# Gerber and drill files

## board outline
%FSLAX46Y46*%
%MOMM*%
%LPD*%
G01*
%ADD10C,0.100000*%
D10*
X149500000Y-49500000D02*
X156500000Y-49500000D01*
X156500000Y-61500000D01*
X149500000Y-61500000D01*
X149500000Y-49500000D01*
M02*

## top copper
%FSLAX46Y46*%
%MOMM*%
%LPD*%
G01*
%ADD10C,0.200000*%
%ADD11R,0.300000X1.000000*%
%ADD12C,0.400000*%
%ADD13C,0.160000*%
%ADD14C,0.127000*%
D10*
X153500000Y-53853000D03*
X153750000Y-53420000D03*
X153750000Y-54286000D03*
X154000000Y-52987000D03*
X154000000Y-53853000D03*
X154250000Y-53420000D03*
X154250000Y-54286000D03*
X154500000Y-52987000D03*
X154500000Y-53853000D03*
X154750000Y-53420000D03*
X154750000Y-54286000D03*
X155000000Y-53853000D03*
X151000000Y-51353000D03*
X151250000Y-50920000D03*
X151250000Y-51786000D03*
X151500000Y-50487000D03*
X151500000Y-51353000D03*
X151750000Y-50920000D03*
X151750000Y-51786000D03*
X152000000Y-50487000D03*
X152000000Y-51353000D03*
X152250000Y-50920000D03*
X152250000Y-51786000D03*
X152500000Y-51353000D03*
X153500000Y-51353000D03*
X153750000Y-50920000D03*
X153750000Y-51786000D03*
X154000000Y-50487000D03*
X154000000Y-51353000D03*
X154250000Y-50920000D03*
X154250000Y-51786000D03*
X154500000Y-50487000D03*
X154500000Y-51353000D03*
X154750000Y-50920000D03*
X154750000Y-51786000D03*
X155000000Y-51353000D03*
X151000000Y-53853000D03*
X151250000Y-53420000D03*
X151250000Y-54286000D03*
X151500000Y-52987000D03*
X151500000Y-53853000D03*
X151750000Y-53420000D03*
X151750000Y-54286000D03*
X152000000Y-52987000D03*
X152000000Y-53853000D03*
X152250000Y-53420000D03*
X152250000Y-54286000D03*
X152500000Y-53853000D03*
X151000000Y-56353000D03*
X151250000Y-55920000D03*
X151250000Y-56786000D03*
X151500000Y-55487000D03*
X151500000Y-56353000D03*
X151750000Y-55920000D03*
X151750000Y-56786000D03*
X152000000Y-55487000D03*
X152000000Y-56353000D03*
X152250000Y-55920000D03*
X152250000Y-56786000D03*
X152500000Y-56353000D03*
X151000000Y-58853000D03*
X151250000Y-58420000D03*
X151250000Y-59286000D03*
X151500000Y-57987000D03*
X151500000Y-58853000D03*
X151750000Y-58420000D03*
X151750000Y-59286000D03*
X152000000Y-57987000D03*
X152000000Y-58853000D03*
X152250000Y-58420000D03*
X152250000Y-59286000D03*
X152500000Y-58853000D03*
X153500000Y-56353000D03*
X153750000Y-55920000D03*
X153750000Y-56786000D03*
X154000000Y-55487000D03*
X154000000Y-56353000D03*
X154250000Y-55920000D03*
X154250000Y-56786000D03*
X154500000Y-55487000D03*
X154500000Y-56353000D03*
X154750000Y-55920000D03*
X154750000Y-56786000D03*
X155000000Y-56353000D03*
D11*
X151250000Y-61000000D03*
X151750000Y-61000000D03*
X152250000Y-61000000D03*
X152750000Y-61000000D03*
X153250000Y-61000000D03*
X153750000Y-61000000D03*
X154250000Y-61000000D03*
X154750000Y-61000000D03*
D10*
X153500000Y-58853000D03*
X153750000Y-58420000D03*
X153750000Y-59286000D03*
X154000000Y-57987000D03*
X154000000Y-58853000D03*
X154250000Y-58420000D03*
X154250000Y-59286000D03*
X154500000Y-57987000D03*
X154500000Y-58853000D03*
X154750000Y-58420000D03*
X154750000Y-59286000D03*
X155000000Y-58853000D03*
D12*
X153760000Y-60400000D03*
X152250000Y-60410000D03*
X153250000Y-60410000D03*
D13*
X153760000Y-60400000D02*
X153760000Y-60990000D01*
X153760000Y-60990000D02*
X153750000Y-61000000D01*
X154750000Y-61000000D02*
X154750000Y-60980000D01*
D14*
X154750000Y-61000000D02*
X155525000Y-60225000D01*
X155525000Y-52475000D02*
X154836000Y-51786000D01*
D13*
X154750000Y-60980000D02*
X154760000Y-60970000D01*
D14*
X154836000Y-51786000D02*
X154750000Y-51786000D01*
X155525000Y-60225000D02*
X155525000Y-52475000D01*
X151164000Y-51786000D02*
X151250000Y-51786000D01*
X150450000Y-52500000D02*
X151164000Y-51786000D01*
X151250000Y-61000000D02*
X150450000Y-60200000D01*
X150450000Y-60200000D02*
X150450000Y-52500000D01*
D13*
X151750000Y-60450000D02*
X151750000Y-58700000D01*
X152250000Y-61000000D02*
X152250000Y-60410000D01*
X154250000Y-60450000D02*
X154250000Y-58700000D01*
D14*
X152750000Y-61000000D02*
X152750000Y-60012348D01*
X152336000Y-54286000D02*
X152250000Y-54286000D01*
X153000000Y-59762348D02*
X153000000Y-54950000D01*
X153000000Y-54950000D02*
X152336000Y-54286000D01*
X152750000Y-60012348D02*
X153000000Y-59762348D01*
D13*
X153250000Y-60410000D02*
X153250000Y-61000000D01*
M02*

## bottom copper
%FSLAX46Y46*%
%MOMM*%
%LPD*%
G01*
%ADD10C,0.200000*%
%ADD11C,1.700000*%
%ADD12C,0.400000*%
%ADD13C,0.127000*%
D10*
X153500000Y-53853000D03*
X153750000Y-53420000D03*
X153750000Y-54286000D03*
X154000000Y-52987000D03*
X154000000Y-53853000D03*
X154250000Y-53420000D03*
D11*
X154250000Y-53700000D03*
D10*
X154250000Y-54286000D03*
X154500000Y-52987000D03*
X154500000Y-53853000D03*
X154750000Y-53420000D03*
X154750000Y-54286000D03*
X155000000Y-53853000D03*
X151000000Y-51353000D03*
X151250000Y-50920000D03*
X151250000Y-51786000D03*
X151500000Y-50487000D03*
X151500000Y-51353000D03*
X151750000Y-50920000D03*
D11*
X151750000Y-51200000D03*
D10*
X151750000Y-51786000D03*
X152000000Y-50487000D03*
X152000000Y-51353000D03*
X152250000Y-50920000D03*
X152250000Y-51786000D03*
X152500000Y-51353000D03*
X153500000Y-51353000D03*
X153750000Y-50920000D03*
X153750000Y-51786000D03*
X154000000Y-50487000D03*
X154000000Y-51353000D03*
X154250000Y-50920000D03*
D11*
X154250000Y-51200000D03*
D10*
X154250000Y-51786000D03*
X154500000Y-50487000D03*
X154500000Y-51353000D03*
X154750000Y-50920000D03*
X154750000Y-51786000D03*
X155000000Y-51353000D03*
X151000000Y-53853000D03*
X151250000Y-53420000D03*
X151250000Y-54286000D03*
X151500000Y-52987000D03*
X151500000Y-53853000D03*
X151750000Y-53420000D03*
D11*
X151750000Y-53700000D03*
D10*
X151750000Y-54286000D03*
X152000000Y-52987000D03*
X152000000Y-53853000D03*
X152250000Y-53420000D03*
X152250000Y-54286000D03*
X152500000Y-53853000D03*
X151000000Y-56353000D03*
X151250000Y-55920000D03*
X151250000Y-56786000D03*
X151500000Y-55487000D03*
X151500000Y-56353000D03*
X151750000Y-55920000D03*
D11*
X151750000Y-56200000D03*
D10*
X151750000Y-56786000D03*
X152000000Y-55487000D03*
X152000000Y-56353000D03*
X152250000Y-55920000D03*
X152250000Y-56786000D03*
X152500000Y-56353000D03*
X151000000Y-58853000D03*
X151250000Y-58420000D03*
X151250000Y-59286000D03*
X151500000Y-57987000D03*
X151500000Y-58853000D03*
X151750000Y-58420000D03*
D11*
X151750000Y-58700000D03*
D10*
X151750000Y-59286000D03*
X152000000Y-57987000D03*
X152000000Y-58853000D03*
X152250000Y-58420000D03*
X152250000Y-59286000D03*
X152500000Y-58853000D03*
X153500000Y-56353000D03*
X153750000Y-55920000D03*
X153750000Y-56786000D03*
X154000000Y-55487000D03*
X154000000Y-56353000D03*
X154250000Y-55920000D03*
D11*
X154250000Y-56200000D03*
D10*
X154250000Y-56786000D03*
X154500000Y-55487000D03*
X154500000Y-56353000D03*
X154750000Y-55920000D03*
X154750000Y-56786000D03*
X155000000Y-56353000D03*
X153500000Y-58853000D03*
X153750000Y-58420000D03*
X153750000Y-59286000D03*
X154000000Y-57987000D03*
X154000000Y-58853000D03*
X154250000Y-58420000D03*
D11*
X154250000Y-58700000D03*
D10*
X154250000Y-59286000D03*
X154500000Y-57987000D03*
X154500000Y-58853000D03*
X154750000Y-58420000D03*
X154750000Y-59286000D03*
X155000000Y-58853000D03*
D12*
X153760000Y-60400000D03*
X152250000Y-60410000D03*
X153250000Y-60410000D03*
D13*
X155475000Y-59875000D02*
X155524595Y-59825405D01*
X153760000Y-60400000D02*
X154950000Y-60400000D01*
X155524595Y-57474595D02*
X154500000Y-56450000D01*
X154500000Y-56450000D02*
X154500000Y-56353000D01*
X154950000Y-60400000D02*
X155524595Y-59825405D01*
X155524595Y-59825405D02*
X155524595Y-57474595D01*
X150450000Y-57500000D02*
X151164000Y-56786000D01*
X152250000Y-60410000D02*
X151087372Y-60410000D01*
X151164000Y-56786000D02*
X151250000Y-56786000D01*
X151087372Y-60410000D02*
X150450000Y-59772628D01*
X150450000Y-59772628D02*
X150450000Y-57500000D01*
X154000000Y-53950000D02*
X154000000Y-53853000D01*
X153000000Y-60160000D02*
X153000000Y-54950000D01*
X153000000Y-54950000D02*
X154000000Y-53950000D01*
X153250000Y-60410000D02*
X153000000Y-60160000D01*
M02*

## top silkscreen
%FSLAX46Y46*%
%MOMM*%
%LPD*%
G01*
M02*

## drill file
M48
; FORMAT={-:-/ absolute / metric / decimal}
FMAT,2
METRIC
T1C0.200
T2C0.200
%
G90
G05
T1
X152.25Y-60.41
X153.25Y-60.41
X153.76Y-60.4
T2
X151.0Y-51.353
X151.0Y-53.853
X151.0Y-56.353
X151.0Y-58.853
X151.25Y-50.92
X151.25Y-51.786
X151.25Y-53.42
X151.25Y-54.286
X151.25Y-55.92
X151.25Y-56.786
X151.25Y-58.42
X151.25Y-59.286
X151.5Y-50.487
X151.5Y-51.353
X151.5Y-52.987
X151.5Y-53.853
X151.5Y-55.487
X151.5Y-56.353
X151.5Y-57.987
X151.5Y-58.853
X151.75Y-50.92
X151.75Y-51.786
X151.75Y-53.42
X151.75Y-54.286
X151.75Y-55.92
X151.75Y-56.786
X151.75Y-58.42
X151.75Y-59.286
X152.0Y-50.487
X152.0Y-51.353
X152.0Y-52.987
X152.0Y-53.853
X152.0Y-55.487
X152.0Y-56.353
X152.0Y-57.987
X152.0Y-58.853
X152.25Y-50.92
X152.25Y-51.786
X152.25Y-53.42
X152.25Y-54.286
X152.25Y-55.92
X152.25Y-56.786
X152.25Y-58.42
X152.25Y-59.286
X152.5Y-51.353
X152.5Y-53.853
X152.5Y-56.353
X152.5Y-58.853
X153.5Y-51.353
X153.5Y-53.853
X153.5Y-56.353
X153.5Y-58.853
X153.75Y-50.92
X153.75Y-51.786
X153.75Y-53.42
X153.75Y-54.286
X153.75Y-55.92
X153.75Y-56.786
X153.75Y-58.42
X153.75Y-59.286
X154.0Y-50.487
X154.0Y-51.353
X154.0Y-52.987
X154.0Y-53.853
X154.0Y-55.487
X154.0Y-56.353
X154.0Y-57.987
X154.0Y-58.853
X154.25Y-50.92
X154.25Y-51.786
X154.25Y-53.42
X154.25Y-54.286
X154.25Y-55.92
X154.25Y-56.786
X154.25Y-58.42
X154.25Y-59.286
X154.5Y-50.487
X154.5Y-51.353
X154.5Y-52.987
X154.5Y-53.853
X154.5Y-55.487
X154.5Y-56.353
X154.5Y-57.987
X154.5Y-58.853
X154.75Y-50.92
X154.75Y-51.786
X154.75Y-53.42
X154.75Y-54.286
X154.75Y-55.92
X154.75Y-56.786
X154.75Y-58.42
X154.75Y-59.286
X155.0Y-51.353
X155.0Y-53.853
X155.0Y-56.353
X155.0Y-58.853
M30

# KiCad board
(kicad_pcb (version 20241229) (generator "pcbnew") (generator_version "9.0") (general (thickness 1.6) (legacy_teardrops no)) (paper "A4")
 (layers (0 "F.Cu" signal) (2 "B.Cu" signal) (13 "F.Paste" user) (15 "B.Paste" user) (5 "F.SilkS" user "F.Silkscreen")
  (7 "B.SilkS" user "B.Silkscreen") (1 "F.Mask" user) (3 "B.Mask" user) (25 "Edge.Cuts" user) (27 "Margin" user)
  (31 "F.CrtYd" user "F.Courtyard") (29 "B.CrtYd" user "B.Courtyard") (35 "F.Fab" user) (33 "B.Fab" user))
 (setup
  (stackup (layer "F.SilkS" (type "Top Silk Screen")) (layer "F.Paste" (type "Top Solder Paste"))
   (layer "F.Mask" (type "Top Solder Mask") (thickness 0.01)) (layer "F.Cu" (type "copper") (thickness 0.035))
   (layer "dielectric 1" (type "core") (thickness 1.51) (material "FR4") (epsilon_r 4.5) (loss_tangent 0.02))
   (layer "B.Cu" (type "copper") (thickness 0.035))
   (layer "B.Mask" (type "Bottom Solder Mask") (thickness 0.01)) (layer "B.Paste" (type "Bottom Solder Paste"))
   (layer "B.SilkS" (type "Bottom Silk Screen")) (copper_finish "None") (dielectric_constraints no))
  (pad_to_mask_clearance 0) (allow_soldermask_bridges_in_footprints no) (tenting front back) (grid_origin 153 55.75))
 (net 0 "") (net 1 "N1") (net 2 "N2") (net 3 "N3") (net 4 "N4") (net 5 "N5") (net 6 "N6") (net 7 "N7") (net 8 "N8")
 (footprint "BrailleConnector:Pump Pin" (layer "F.Cu") (at 154.25 53.7)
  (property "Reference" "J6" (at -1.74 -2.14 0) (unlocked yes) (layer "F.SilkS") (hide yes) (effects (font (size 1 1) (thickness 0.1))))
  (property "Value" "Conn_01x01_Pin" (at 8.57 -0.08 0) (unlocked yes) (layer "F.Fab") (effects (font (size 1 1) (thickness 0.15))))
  (pad "1" thru_hole circle (at -0.75 0.153) (size 0.2 0.2) (drill 0.2) (layers "*.Cu" "*.Mask") (remove_unused_layers no) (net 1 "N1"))
  (pad "1" thru_hole circle (at -0.5 -0.28) (size 0.2 0.2) (drill 0.2) (layers "*.Cu" "*.Mask") (remove_unused_layers no) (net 1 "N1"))
  (pad "1" thru_hole circle (at -0.5 0.586) (size 0.2 0.2) (drill 0.2) (layers "*.Cu" "*.Mask") (remove_unused_layers no) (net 1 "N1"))
  (pad "1" thru_hole circle (at -0.25 -0.713) (size 0.2 0.2) (drill 0.2) (layers "*.Cu" "*.Mask") (remove_unused_layers no) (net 1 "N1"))
  (pad "1" thru_hole circle (at -0.25 0.153) (size 0.2 0.2) (drill 0.2) (layers "*.Cu" "*.Mask") (remove_unused_layers no) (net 1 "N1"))
  (pad "1" thru_hole circle (at 0 -0.28) (size 0.2 0.2) (drill 0.2) (layers "*.Cu" "*.Mask") (remove_unused_layers no) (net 1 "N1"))
  (pad "1" smd circle (at 0 0) (size 1.7 1.7) (layers "B.Cu" "B.Mask") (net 1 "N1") (solder_mask_margin 0) (solder_paste_margin 0)
   (clearance 0))
  (pad "1" thru_hole circle (at 0 0.586) (size 0.2 0.2) (drill 0.2) (layers "*.Cu" "*.Mask") (remove_unused_layers no) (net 1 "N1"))
  (pad "1" thru_hole circle (at 0.25 -0.713) (size 0.2 0.2) (drill 0.2) (layers "*.Cu" "*.Mask") (remove_unused_layers no) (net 1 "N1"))
  (pad "1" thru_hole circle (at 0.25 0.153) (size 0.2 0.2) (drill 0.2) (layers "*.Cu" "*.Mask") (remove_unused_layers no) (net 1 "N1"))
  (pad "1" thru_hole circle (at 0.5 -0.28) (size 0.2 0.2) (drill 0.2) (layers "*.Cu" "*.Mask") (remove_unused_layers no) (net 1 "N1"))
  (pad "1" thru_hole circle (at 0.5 0.586) (size 0.2 0.2) (drill 0.2) (layers "*.Cu" "*.Mask") (remove_unused_layers no) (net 1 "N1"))
  (pad "1" thru_hole circle (at 0.75 0.153) (size 0.2 0.2) (drill 0.2) (layers "*.Cu" "*.Mask") (remove_unused_layers no) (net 1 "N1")))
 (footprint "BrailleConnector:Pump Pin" (layer "F.Cu") (at 151.75 51.2)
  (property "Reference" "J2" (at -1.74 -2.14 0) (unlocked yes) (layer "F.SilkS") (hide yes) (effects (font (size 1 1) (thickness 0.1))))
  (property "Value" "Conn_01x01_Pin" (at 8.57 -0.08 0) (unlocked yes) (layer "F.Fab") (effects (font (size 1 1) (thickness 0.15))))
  (pad "1" thru_hole circle (at -0.75 0.153) (size 0.2 0.2) (drill 0.2) (layers "*.Cu" "*.Mask") (remove_unused_layers no) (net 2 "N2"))
  (pad "1" thru_hole circle (at -0.5 -0.28) (size 0.2 0.2) (drill 0.2) (layers "*.Cu" "*.Mask") (remove_unused_layers no) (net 2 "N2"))
  (pad "1" thru_hole circle (at -0.5 0.586) (size 0.2 0.2) (drill 0.2) (layers "*.Cu" "*.Mask") (remove_unused_layers no) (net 2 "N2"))
  (pad "1" thru_hole circle (at -0.25 -0.713) (size 0.2 0.2) (drill 0.2) (layers "*.Cu" "*.Mask") (remove_unused_layers no) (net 2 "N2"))
  (pad "1" thru_hole circle (at -0.25 0.153) (size 0.2 0.2) (drill 0.2) (layers "*.Cu" "*.Mask") (remove_unused_layers no) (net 2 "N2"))
  (pad "1" thru_hole circle (at 0 -0.28) (size 0.2 0.2) (drill 0.2) (layers "*.Cu" "*.Mask") (remove_unused_layers no) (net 2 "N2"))
  (pad "1" smd circle (at 0 0) (size 1.7 1.7) (layers "B.Cu" "B.Mask") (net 2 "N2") (solder_mask_margin 0) (solder_paste_margin 0)
   (clearance 0))
  (pad "1" thru_hole circle (at 0 0.586) (size 0.2 0.2) (drill 0.2) (layers "*.Cu" "*.Mask") (remove_unused_layers no) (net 2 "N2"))
  (pad "1" thru_hole circle (at 0.25 -0.713) (size 0.2 0.2) (drill 0.2) (layers "*.Cu" "*.Mask") (remove_unused_layers no) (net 2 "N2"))
  (pad "1" thru_hole circle (at 0.25 0.153) (size 0.2 0.2) (drill 0.2) (layers "*.Cu" "*.Mask") (remove_unused_layers no) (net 2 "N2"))
  (pad "1" thru_hole circle (at 0.5 -0.28) (size 0.2 0.2) (drill 0.2) (layers "*.Cu" "*.Mask") (remove_unused_layers no) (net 2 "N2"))
  (pad "1" thru_hole circle (at 0.5 0.586) (size 0.2 0.2) (drill 0.2) (layers "*.Cu" "*.Mask") (remove_unused_layers no) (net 2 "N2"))
  (pad "1" thru_hole circle (at 0.75 0.153) (size 0.2 0.2) (drill 0.2) (layers "*.Cu" "*.Mask") (remove_unused_layers no) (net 2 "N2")))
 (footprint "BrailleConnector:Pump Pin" (layer "F.Cu") (at 154.25 51.2)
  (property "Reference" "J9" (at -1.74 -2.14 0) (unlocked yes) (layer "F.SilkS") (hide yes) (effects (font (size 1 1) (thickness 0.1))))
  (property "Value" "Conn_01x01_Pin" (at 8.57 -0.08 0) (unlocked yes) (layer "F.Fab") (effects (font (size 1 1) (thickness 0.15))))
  (pad "1" thru_hole circle (at -0.75 0.153) (size 0.2 0.2) (drill 0.2) (layers "*.Cu" "*.Mask") (remove_unused_layers no) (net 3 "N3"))
  (pad "1" thru_hole circle (at -0.5 -0.28) (size 0.2 0.2) (drill 0.2) (layers "*.Cu" "*.Mask") (remove_unused_layers no) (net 3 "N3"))
  (pad "1" thru_hole circle (at -0.5 0.586) (size 0.2 0.2) (drill 0.2) (layers "*.Cu" "*.Mask") (remove_unused_layers no) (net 3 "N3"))
  (pad "1" thru_hole circle (at -0.25 -0.713) (size 0.2 0.2) (drill 0.2) (layers "*.Cu" "*.Mask") (remove_unused_layers no) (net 3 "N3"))
  (pad "1" thru_hole circle (at -0.25 0.153) (size 0.2 0.2) (drill 0.2) (layers "*.Cu" "*.Mask") (remove_unused_layers no) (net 3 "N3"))
  (pad "1" thru_hole circle (at 0 -0.28) (size 0.2 0.2) (drill 0.2) (layers "*.Cu" "*.Mask") (remove_unused_layers no) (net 3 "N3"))
  (pad "1" smd circle (at 0 0) (size 1.7 1.7) (layers "B.Cu" "B.Mask") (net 3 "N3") (solder_mask_margin 0) (solder_paste_margin 0)
   (clearance 0))
  (pad "1" thru_hole circle (at 0 0.586) (size 0.2 0.2) (drill 0.2) (layers "*.Cu" "*.Mask") (remove_unused_layers no) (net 3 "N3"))
  (pad "1" thru_hole circle (at 0.25 -0.713) (size 0.2 0.2) (drill 0.2) (layers "*.Cu" "*.Mask") (remove_unused_layers no) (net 3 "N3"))
  (pad "1" thru_hole circle (at 0.25 0.153) (size 0.2 0.2) (drill 0.2) (layers "*.Cu" "*.Mask") (remove_unused_layers no) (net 3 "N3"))
  (pad "1" thru_hole circle (at 0.5 -0.28) (size 0.2 0.2) (drill 0.2) (layers "*.Cu" "*.Mask") (remove_unused_layers no) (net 3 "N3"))
  (pad "1" thru_hole circle (at 0.5 0.586) (size 0.2 0.2) (drill 0.2) (layers "*.Cu" "*.Mask") (remove_unused_layers no) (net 3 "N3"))
  (pad "1" thru_hole circle (at 0.75 0.153) (size 0.2 0.2) (drill 0.2) (layers "*.Cu" "*.Mask") (remove_unused_layers no) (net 3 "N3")))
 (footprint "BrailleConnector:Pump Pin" (layer "F.Cu") (at 151.75 53.7)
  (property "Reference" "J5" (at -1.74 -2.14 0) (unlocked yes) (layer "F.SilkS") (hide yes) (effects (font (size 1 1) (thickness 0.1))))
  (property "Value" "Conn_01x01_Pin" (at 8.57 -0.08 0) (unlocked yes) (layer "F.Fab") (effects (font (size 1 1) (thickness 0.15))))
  (pad "1" thru_hole circle (at -0.75 0.153) (size 0.2 0.2) (drill 0.2) (layers "*.Cu" "*.Mask") (remove_unused_layers no) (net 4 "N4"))
  (pad "1" thru_hole circle (at -0.5 -0.28) (size 0.2 0.2) (drill 0.2) (layers "*.Cu" "*.Mask") (remove_unused_layers no) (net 4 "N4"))
  (pad "1" thru_hole circle (at -0.5 0.586) (size 0.2 0.2) (drill 0.2) (layers "*.Cu" "*.Mask") (remove_unused_layers no) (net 4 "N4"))
  (pad "1" thru_hole circle (at -0.25 -0.713) (size 0.2 0.2) (drill 0.2) (layers "*.Cu" "*.Mask") (remove_unused_layers no) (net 4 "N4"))
  (pad "1" thru_hole circle (at -0.25 0.153) (size 0.2 0.2) (drill 0.2) (layers "*.Cu" "*.Mask") (remove_unused_layers no) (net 4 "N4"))
  (pad "1" thru_hole circle (at 0 -0.28) (size 0.2 0.2) (drill 0.2) (layers "*.Cu" "*.Mask") (remove_unused_layers no) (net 4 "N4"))
  (pad "1" smd circle (at 0 0) (size 1.7 1.7) (layers "B.Cu" "B.Mask") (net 4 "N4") (solder_mask_margin 0) (solder_paste_margin 0)
   (clearance 0))
  (pad "1" thru_hole circle (at 0 0.586) (size 0.2 0.2) (drill 0.2) (layers "*.Cu" "*.Mask") (remove_unused_layers no) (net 4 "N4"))
  (pad "1" thru_hole circle (at 0.25 -0.713) (size 0.2 0.2) (drill 0.2) (layers "*.Cu" "*.Mask") (remove_unused_layers no) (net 4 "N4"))
  (pad "1" thru_hole circle (at 0.25 0.153) (size 0.2 0.2) (drill 0.2) (layers "*.Cu" "*.Mask") (remove_unused_layers no) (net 4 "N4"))
  (pad "1" thru_hole circle (at 0.5 -0.28) (size 0.2 0.2) (drill 0.2) (layers "*.Cu" "*.Mask") (remove_unused_layers no) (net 4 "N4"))
  (pad "1" thru_hole circle (at 0.5 0.586) (size 0.2 0.2) (drill 0.2) (layers "*.Cu" "*.Mask") (remove_unused_layers no) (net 4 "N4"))
  (pad "1" thru_hole circle (at 0.75 0.153) (size 0.2 0.2) (drill 0.2) (layers "*.Cu" "*.Mask") (remove_unused_layers no) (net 4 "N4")))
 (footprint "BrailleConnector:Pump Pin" (layer "F.Cu") (at 151.75 56.2)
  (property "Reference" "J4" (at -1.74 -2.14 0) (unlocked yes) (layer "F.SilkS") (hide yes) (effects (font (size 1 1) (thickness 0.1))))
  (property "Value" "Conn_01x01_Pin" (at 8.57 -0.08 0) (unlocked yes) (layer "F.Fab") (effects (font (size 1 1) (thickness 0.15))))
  (pad "1" thru_hole circle (at -0.75 0.153) (size 0.2 0.2) (drill 0.2) (layers "*.Cu" "*.Mask") (remove_unused_layers no) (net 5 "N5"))
  (pad "1" thru_hole circle (at -0.5 -0.28) (size 0.2 0.2) (drill 0.2) (layers "*.Cu" "*.Mask") (remove_unused_layers no) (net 5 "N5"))
  (pad "1" thru_hole circle (at -0.5 0.586) (size 0.2 0.2) (drill 0.2) (layers "*.Cu" "*.Mask") (remove_unused_layers no) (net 5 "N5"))
  (pad "1" thru_hole circle (at -0.25 -0.713) (size 0.2 0.2) (drill 0.2) (layers "*.Cu" "*.Mask") (remove_unused_layers no) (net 5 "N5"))
  (pad "1" thru_hole circle (at -0.25 0.153) (size 0.2 0.2) (drill 0.2) (layers "*.Cu" "*.Mask") (remove_unused_layers no) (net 5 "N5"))
  (pad "1" thru_hole circle (at 0 -0.28) (size 0.2 0.2) (drill 0.2) (layers "*.Cu" "*.Mask") (remove_unused_layers no) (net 5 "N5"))
  (pad "1" smd circle (at 0 0) (size 1.7 1.7) (layers "B.Cu" "B.Mask") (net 5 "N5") (solder_mask_margin 0) (solder_paste_margin 0)
   (clearance 0))
  (pad "1" thru_hole circle (at 0 0.586) (size 0.2 0.2) (drill 0.2) (layers "*.Cu" "*.Mask") (remove_unused_layers no) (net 5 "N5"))
  (pad "1" thru_hole circle (at 0.25 -0.713) (size 0.2 0.2) (drill 0.2) (layers "*.Cu" "*.Mask") (remove_unused_layers no) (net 5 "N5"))
  (pad "1" thru_hole circle (at 0.25 0.153) (size 0.2 0.2) (drill 0.2) (layers "*.Cu" "*.Mask") (remove_unused_layers no) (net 5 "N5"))
  (pad "1" thru_hole circle (at 0.5 -0.28) (size 0.2 0.2) (drill 0.2) (layers "*.Cu" "*.Mask") (remove_unused_layers no) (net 5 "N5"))
  (pad "1" thru_hole circle (at 0.5 0.586) (size 0.2 0.2) (drill 0.2) (layers "*.Cu" "*.Mask") (remove_unused_layers no) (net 5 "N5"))
  (pad "1" thru_hole circle (at 0.75 0.153) (size 0.2 0.2) (drill 0.2) (layers "*.Cu" "*.Mask") (remove_unused_layers no) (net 5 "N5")))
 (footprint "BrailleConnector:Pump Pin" (layer "F.Cu") (at 151.75 58.7)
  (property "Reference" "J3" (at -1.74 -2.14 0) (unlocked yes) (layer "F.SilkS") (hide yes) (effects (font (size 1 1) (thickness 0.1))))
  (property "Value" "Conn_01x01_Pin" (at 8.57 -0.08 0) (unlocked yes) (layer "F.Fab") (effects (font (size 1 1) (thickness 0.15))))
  (pad "1" thru_hole circle (at -0.75 0.153) (size 0.2 0.2) (drill 0.2) (layers "*.Cu" "*.Mask") (remove_unused_layers no) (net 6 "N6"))
  (pad "1" thru_hole circle (at -0.5 -0.28) (size 0.2 0.2) (drill 0.2) (layers "*.Cu" "*.Mask") (remove_unused_layers no) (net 6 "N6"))
  (pad "1" thru_hole circle (at -0.5 0.586) (size 0.2 0.2) (drill 0.2) (layers "*.Cu" "*.Mask") (remove_unused_layers no) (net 6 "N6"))
  (pad "1" thru_hole circle (at -0.25 -0.713) (size 0.2 0.2) (drill 0.2) (layers "*.Cu" "*.Mask") (remove_unused_layers no) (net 6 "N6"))
  (pad "1" thru_hole circle (at -0.25 0.153) (size 0.2 0.2) (drill 0.2) (layers "*.Cu" "*.Mask") (remove_unused_layers no) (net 6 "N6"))
  (pad "1" thru_hole circle (at 0 -0.28) (size 0.2 0.2) (drill 0.2) (layers "*.Cu" "*.Mask") (remove_unused_layers no) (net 6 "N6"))
  (pad "1" smd circle (at 0 0) (size 1.7 1.7) (layers "B.Cu" "B.Mask") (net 6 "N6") (solder_mask_margin 0) (solder_paste_margin 0)
   (clearance 0))
  (pad "1" thru_hole circle (at 0 0.586) (size 0.2 0.2) (drill 0.2) (layers "*.Cu" "*.Mask") (remove_unused_layers no) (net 6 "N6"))
  (pad "1" thru_hole circle (at 0.25 -0.713) (size 0.2 0.2) (drill 0.2) (layers "*.Cu" "*.Mask") (remove_unused_layers no) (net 6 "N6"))
  (pad "1" thru_hole circle (at 0.25 0.153) (size 0.2 0.2) (drill 0.2) (layers "*.Cu" "*.Mask") (remove_unused_layers no) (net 6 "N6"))
  (pad "1" thru_hole circle (at 0.5 -0.28) (size 0.2 0.2) (drill 0.2) (layers "*.Cu" "*.Mask") (remove_unused_layers no) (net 6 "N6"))
  (pad "1" thru_hole circle (at 0.5 0.586) (size 0.2 0.2) (drill 0.2) (layers "*.Cu" "*.Mask") (remove_unused_layers no) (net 6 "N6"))
  (pad "1" thru_hole circle (at 0.75 0.153) (size 0.2 0.2) (drill 0.2) (layers "*.Cu" "*.Mask") (remove_unused_layers no) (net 6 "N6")))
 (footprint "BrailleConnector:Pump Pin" (layer "F.Cu") (at 154.25 56.2)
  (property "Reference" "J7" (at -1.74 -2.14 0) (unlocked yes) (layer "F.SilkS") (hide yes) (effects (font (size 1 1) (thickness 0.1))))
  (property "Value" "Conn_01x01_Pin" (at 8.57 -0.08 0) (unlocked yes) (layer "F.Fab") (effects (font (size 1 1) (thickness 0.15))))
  (pad "1" thru_hole circle (at -0.75 0.153) (size 0.2 0.2) (drill 0.2) (layers "*.Cu" "*.Mask") (remove_unused_layers no) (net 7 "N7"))
  (pad "1" thru_hole circle (at -0.5 -0.28) (size 0.2 0.2) (drill 0.2) (layers "*.Cu" "*.Mask") (remove_unused_layers no) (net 7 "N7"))
  (pad "1" thru_hole circle (at -0.5 0.586) (size 0.2 0.2) (drill 0.2) (layers "*.Cu" "*.Mask") (remove_unused_layers no) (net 7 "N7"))
  (pad "1" thru_hole circle (at -0.25 -0.713) (size 0.2 0.2) (drill 0.2) (layers "*.Cu" "*.Mask") (remove_unused_layers no) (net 7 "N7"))
  (pad "1" thru_hole circle (at -0.25 0.153) (size 0.2 0.2) (drill 0.2) (layers "*.Cu" "*.Mask") (remove_unused_layers no) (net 7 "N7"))
  (pad "1" thru_hole circle (at 0 -0.28) (size 0.2 0.2) (drill 0.2) (layers "*.Cu" "*.Mask") (remove_unused_layers no) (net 7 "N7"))
  (pad "1" smd circle (at 0 0) (size 1.7 1.7) (layers "B.Cu" "B.Mask") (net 7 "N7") (solder_mask_margin 0) (solder_paste_margin 0)
   (clearance 0))
  (pad "1" thru_hole circle (at 0 0.586) (size 0.2 0.2) (drill 0.2) (layers "*.Cu" "*.Mask") (remove_unused_layers no) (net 7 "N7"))
  (pad "1" thru_hole circle (at 0.25 -0.713) (size 0.2 0.2) (drill 0.2) (layers "*.Cu" "*.Mask") (remove_unused_layers no) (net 7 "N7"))
  (pad "1" thru_hole circle (at 0.25 0.153) (size 0.2 0.2) (drill 0.2) (layers "*.Cu" "*.Mask") (remove_unused_layers no) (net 7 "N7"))
  (pad "1" thru_hole circle (at 0.5 -0.28) (size 0.2 0.2) (drill 0.2) (layers "*.Cu" "*.Mask") (remove_unused_layers no) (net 7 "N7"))
  (pad "1" thru_hole circle (at 0.5 0.586) (size 0.2 0.2) (drill 0.2) (layers "*.Cu" "*.Mask") (remove_unused_layers no) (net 7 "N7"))
  (pad "1" thru_hole circle (at 0.75 0.153) (size 0.2 0.2) (drill 0.2) (layers "*.Cu" "*.Mask") (remove_unused_layers no) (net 7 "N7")))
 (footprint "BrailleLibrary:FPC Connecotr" (layer "F.Cu") (at 153 61 90)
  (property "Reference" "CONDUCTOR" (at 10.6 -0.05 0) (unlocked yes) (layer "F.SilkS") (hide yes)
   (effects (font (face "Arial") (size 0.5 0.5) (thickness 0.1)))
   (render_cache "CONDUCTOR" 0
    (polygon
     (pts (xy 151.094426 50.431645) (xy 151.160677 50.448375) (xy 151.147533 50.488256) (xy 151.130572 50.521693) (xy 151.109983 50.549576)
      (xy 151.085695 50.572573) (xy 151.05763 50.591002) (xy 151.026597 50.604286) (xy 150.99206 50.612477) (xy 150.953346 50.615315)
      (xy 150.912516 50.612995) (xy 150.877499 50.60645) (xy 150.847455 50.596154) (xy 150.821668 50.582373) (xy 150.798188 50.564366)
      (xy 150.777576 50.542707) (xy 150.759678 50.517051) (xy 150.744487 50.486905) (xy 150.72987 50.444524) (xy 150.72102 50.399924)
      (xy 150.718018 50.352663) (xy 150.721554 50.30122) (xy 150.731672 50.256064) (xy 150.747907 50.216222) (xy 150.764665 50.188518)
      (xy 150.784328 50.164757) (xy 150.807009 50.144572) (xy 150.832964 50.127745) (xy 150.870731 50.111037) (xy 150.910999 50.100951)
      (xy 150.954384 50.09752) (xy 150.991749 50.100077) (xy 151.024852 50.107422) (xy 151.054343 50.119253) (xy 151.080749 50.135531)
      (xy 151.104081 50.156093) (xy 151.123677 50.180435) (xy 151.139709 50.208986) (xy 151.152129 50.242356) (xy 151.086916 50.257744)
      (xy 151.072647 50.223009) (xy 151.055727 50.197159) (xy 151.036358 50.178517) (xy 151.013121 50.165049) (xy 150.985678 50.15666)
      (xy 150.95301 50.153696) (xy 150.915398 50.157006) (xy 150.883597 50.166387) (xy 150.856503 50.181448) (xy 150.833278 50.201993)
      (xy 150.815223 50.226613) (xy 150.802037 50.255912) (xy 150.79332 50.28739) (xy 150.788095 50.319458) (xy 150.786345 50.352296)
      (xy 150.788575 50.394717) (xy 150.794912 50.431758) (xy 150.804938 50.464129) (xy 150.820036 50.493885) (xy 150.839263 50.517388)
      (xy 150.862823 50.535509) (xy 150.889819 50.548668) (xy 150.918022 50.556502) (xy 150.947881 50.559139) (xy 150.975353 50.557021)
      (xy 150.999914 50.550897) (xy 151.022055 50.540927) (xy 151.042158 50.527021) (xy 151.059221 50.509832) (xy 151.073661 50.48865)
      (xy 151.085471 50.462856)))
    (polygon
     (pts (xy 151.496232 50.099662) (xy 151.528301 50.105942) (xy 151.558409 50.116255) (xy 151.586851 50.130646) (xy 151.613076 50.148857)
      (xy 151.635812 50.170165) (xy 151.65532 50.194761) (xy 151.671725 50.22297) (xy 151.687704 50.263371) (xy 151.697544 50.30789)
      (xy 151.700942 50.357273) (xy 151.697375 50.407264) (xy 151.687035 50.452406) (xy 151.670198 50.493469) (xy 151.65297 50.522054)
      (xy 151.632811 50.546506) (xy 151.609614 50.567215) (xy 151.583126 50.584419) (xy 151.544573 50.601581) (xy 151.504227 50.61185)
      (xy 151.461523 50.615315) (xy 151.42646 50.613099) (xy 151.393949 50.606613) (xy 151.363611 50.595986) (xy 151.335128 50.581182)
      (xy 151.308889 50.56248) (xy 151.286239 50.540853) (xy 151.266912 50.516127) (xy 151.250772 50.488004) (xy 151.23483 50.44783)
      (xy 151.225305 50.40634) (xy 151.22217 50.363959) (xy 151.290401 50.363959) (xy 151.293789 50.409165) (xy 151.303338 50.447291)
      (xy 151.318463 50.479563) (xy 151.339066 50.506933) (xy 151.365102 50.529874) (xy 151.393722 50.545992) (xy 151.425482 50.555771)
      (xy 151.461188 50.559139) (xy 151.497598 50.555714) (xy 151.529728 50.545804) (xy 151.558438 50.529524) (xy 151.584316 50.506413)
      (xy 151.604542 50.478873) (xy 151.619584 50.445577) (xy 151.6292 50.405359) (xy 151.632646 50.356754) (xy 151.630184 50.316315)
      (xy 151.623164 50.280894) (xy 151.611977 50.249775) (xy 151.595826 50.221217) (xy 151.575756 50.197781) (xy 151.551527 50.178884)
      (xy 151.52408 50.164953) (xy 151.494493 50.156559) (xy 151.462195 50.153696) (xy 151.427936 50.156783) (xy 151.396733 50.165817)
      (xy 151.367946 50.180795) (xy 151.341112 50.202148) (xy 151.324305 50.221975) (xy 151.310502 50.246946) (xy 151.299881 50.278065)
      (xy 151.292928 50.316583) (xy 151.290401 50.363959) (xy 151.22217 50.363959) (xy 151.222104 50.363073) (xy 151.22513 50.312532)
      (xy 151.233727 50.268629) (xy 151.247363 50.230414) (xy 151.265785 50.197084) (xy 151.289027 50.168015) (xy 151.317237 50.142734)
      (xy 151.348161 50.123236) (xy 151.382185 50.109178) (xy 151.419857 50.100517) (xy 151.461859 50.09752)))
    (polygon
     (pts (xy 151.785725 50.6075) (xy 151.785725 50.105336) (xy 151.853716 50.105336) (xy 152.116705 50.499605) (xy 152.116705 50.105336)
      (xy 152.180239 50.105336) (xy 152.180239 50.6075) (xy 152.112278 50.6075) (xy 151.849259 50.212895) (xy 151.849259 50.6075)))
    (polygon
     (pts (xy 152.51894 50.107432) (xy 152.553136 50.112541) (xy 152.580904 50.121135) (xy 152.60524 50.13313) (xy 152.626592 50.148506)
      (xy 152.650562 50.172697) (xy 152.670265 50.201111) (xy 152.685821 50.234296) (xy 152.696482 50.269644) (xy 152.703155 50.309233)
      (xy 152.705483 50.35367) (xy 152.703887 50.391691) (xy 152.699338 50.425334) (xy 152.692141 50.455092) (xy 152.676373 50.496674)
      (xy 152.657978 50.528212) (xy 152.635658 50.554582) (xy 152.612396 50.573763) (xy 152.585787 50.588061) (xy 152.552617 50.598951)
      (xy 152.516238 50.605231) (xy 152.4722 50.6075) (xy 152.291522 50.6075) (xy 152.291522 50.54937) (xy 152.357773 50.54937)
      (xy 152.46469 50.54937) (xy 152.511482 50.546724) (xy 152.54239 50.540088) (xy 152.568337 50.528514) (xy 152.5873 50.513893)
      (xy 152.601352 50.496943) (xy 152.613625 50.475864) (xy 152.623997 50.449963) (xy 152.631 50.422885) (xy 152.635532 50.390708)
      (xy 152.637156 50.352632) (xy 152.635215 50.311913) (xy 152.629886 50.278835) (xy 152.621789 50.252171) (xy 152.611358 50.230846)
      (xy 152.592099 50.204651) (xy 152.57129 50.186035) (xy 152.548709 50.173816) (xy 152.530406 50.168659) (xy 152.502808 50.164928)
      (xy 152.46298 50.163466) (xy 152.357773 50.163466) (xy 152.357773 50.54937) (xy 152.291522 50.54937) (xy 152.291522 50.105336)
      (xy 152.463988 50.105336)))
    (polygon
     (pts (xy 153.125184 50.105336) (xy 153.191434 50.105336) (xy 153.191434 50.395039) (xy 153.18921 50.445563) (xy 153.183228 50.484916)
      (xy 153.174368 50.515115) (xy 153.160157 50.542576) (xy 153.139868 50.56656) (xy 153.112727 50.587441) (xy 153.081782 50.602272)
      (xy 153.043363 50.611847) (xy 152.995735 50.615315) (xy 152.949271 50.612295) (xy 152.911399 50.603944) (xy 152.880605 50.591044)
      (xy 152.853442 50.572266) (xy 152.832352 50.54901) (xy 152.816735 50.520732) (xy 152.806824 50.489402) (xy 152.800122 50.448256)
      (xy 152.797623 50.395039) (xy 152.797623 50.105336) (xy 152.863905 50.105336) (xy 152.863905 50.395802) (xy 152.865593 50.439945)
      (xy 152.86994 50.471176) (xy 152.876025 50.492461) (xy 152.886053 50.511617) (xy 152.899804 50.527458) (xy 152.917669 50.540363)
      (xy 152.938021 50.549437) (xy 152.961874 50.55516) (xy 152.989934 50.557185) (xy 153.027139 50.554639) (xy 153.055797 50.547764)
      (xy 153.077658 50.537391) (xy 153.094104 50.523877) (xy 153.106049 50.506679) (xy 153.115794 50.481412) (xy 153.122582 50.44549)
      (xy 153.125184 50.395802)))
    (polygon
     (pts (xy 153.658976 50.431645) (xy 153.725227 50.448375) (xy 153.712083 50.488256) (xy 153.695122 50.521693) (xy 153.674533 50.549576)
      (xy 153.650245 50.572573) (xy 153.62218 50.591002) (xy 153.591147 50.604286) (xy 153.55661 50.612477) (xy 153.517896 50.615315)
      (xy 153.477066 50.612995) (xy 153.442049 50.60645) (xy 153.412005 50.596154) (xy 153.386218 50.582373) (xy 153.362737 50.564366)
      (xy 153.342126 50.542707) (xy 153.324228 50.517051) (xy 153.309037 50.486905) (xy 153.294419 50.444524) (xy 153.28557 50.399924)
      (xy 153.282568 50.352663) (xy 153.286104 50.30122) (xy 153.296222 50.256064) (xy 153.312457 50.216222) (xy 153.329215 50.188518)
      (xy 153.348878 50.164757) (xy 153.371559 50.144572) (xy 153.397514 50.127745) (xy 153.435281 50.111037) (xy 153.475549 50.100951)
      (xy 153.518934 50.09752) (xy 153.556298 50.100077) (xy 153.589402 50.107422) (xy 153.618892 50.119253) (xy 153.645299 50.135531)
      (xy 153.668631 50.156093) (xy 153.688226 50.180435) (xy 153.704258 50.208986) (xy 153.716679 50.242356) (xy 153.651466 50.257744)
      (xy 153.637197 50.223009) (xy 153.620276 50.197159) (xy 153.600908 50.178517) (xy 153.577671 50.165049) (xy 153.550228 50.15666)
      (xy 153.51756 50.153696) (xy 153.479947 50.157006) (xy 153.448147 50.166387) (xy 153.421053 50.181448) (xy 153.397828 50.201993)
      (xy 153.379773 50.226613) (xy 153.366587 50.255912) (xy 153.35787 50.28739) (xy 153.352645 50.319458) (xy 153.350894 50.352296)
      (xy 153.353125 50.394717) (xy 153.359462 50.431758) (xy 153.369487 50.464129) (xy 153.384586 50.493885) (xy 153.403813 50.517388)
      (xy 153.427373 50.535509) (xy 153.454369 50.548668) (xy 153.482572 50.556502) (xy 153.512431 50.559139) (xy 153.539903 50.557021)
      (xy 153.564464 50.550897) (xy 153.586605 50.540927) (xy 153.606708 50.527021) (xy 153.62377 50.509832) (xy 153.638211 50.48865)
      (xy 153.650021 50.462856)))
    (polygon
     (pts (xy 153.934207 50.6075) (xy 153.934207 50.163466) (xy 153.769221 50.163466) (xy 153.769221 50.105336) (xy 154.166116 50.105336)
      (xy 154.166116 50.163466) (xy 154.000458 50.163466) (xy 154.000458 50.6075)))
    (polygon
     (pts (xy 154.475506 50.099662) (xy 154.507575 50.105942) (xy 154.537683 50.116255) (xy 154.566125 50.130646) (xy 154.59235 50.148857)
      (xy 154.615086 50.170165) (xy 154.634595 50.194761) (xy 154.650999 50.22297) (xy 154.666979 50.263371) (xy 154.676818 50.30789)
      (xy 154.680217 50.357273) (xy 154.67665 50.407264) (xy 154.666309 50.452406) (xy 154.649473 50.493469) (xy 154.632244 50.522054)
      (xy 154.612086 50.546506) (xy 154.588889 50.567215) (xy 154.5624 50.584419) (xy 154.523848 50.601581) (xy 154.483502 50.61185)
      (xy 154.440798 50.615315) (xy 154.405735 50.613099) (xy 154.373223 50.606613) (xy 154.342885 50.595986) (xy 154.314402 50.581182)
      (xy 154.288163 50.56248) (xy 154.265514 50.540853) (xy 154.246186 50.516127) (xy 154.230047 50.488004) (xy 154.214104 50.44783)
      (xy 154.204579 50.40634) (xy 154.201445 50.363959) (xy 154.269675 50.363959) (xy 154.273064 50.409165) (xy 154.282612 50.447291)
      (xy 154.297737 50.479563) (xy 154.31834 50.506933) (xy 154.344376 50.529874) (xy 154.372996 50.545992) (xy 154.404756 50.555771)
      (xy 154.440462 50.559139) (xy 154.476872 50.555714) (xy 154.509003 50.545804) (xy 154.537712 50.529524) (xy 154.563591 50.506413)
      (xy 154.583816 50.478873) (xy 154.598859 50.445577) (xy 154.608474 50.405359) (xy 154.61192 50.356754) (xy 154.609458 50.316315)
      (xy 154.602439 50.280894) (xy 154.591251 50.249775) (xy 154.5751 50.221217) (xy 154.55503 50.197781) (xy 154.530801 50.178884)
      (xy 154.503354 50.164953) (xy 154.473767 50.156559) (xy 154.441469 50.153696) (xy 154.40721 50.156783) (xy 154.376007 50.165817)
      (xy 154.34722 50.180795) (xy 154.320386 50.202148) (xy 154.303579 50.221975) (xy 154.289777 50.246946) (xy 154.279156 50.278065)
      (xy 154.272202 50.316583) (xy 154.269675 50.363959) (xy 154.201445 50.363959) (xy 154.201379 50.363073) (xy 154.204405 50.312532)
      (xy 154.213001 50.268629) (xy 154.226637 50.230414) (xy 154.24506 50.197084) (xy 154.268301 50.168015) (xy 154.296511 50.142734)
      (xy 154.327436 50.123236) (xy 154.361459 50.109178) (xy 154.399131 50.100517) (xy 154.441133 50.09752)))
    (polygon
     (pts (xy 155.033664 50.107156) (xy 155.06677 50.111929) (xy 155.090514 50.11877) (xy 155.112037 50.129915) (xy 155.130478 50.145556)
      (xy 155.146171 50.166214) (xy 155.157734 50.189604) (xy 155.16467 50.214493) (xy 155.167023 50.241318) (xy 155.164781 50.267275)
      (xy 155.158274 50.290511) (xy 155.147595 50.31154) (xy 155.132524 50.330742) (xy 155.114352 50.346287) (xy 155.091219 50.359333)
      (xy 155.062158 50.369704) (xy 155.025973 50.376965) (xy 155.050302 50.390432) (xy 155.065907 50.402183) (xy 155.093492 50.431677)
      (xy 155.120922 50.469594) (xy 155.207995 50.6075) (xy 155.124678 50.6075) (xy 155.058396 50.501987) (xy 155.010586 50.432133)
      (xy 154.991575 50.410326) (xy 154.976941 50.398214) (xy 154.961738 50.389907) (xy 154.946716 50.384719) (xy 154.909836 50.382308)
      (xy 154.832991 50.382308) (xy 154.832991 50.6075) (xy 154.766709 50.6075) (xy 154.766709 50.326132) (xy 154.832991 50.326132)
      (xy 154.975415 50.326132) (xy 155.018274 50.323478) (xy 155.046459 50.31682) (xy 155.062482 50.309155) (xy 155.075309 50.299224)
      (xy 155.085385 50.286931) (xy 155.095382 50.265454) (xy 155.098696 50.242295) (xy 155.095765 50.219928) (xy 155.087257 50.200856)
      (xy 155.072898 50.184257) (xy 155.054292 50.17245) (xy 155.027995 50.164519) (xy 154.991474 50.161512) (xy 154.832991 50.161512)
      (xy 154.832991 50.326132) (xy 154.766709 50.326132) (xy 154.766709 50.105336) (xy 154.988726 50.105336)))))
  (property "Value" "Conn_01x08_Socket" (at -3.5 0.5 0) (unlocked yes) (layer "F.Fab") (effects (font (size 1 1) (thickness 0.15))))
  (pad "1" smd rect (at 0 -1.75 90) (size 1 0.3) (layers "F.Cu" "F.Mask" "F.Paste") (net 2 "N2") (thermal_bridge_angle 45))
  (pad "2" smd rect (at 0 -1.25 90) (size 1 0.3) (layers "F.Cu" "F.Mask" "F.Paste") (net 6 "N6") (thermal_bridge_angle 45))
  (pad "3" smd rect (at 0 -0.75 90) (size 1 0.3) (layers "F.Cu" "F.Mask" "F.Paste") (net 5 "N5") (thermal_bridge_angle 45))
  (pad "4" smd rect (at 0 -0.25 90) (size 1 0.3) (layers "F.Cu" "F.Mask" "F.Paste") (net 4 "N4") (thermal_bridge_angle 45))
  (pad "5" smd rect (at 0 0.25 90) (size 1 0.3) (layers "F.Cu" "F.Mask" "F.Paste") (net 1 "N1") (thermal_bridge_angle 45))
  (pad "6" smd rect (at 0 0.75 90) (size 1 0.3) (layers "F.Cu" "F.Mask" "F.Paste") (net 7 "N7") (thermal_bridge_angle 45))
  (pad "7" smd rect (at 0 1.25 90) (size 1 0.3) (layers "F.Cu" "F.Mask" "F.Paste") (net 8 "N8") (thermal_bridge_angle 45))
  (pad "8" smd rect (at 0 1.75 90) (size 1 0.3) (layers "F.Cu" "F.Mask" "F.Paste") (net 3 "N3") (thermal_bridge_angle 45)))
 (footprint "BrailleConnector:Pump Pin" (layer "F.Cu") (at 154.25 58.7)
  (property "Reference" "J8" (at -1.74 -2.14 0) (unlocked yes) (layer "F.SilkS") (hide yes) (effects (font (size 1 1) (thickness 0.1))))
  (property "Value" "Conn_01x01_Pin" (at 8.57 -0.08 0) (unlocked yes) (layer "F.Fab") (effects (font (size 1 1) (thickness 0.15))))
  (pad "1" thru_hole circle (at -0.75 0.153) (size 0.2 0.2) (drill 0.2) (layers "*.Cu" "*.Mask") (remove_unused_layers no) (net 8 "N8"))
  (pad "1" thru_hole circle (at -0.5 -0.28) (size 0.2 0.2) (drill 0.2) (layers "*.Cu" "*.Mask") (remove_unused_layers no) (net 8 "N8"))
  (pad "1" thru_hole circle (at -0.5 0.586) (size 0.2 0.2) (drill 0.2) (layers "*.Cu" "*.Mask") (remove_unused_layers no) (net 8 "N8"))
  (pad "1" thru_hole circle (at -0.25 -0.713) (size 0.2 0.2) (drill 0.2) (layers "*.Cu" "*.Mask") (remove_unused_layers no) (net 8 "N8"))
  (pad "1" thru_hole circle (at -0.25 0.153) (size 0.2 0.2) (drill 0.2) (layers "*.Cu" "*.Mask") (remove_unused_layers no) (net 8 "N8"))
  (pad "1" thru_hole circle (at 0 -0.28) (size 0.2 0.2) (drill 0.2) (layers "*.Cu" "*.Mask") (remove_unused_layers no) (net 8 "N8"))
  (pad "1" smd circle (at 0 0) (size 1.7 1.7) (layers "B.Cu" "B.Mask") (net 8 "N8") (solder_mask_margin 0) (solder_paste_margin 0)
   (clearance 0))
  (pad "1" thru_hole circle (at 0 0.586) (size 0.2 0.2) (drill 0.2) (layers "*.Cu" "*.Mask") (remove_unused_layers no) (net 8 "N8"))
  (pad "1" thru_hole circle (at 0.25 -0.713) (size 0.2 0.2) (drill 0.2) (layers "*.Cu" "*.Mask") (remove_unused_layers no) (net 8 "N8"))
  (pad "1" thru_hole circle (at 0.25 0.153) (size 0.2 0.2) (drill 0.2) (layers "*.Cu" "*.Mask") (remove_unused_layers no) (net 8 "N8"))
  (pad "1" thru_hole circle (at 0.5 -0.28) (size 0.2 0.2) (drill 0.2) (layers "*.Cu" "*.Mask") (remove_unused_layers no) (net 8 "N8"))
  (pad "1" thru_hole circle (at 0.5 0.586) (size 0.2 0.2) (drill 0.2) (layers "*.Cu" "*.Mask") (remove_unused_layers no) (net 8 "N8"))
  (pad "1" thru_hole circle (at 0.75 0.153) (size 0.2 0.2) (drill 0.2) (layers "*.Cu" "*.Mask") (remove_unused_layers no) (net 8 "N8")))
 (gr_rect (start 149.5 49.5) (end 156.5 61.5) (stroke (width 0.1) (type solid)) (fill no) (layer "Edge.Cuts"))
 (segment (start 153.76 60.4) (end 153.76 60.99) (width 0.16) (layer "F.Cu") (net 7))
 (segment (start 153.76 60.99) (end 153.75 61) (width 0.16) (layer "F.Cu") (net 7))
 (via (at 153.76 60.4) (size 0.4) (drill 0.2) (layers "F.Cu" "B.Cu") (free yes) (tenting front back) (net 7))
 (segment (start 155.475 59.875) (end 155.524595 59.825405) (width 0.127) (layer "B.Cu") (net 7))
 (segment (start 153.76 60.4) (end 154.95 60.4) (width 0.127) (layer "B.Cu") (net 7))
 (segment (start 155.524595 57.474595) (end 154.5 56.45) (width 0.127) (layer "B.Cu") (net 7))
 (segment (start 154.5 56.45) (end 154.5 56.353) (width 0.127) (layer "B.Cu") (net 7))
 (segment (start 154.95 60.4) (end 155.524595 59.825405) (width 0.127) (layer "B.Cu") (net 7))
 (segment (start 155.524595 59.825405) (end 155.524595 57.474595) (width 0.127) (layer "B.Cu") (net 7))
 (segment (start 154.75 61) (end 154.75 60.98) (width 0.16) (layer "F.Cu") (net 3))
 (segment (start 154.75 61) (end 155.525 60.225) (width 0.127) (layer "F.Cu") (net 3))
 (segment (start 155.525 52.475) (end 154.836 51.786) (width 0.127) (layer "F.Cu") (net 3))
 (segment (start 154.75 60.98) (end 154.76 60.97) (width 0.16) (layer "F.Cu") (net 3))
 (segment (start 154.836 51.786) (end 154.75 51.786) (width 0.127) (layer "F.Cu") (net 3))
 (segment (start 155.525 60.225) (end 155.525 52.475) (width 0.127) (layer "F.Cu") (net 3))
 (segment (start 151.164 51.786) (end 151.25 51.786) (width 0.127) (layer "F.Cu") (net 2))
 (segment (start 150.45 52.5) (end 151.164 51.786) (width 0.127) (layer "F.Cu") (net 2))
 (segment (start 151.25 61) (end 150.45 60.2) (width 0.127) (layer "F.Cu") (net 2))
 (segment (start 150.45 60.2) (end 150.45 52.5) (width 0.127) (layer "F.Cu") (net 2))
 (segment (start 151.75 60.45) (end 151.75 58.7) (width 0.16) (layer "F.Cu") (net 6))
 (segment (start 152.25 61) (end 152.25 60.41) (width 0.16) (layer "F.Cu") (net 5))
 (via (at 152.25 60.41) (size 0.4) (drill 0.2) (layers "F.Cu" "B.Cu") (tenting front back) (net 5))
 (segment (start 150.45 57.5) (end 151.164 56.786) (width 0.127) (layer "B.Cu") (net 5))
 (segment (start 152.25 60.41) (end 151.087372 60.41) (width 0.127) (layer "B.Cu") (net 5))
 (segment (start 151.164 56.786) (end 151.25 56.786) (width 0.127) (layer "B.Cu") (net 5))
 (segment (start 151.087372 60.41) (end 150.45 59.772628) (width 0.127) (layer "B.Cu") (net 5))
 (segment (start 150.45 59.772628) (end 150.45 57.5) (width 0.127) (layer "B.Cu") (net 5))
 (segment (start 154.25 60.45) (end 154.25 58.7) (width 0.16) (layer "F.Cu") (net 8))
 (segment (start 152.75 61) (end 152.75 60.012348) (width 0.127) (layer "F.Cu") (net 4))
 (segment (start 152.336 54.286) (end 152.25 54.286) (width 0.127) (layer "F.Cu") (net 4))
 (segment (start 153 59.762348) (end 153 54.95) (width 0.127) (layer "F.Cu") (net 4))
 (segment (start 153 54.95) (end 152.336 54.286) (width 0.127) (layer "F.Cu") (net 4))
 (segment (start 152.75 60.012348) (end 153 59.762348) (width 0.127) (layer "F.Cu") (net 4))
 (segment (start 153.25 60.41) (end 153.25 61) (width 0.16) (layer "F.Cu") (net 1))
 (via (at 153.25 60.41) (size 0.4) (drill 0.2) (layers "F.Cu" "B.Cu") (tenting front back) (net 1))
 (segment (start 154 53.95) (end 154 53.853) (width 0.127) (layer "B.Cu") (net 1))
 (segment (start 153 60.16) (end 153 54.95) (width 0.127) (layer "B.Cu") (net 1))
 (segment (start 153 54.95) (end 154 53.95) (width 0.127) (layer "B.Cu") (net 1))
 (segment (start 153.25 60.41) (end 153 60.16) (width 0.127) (layer "B.Cu") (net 1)))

